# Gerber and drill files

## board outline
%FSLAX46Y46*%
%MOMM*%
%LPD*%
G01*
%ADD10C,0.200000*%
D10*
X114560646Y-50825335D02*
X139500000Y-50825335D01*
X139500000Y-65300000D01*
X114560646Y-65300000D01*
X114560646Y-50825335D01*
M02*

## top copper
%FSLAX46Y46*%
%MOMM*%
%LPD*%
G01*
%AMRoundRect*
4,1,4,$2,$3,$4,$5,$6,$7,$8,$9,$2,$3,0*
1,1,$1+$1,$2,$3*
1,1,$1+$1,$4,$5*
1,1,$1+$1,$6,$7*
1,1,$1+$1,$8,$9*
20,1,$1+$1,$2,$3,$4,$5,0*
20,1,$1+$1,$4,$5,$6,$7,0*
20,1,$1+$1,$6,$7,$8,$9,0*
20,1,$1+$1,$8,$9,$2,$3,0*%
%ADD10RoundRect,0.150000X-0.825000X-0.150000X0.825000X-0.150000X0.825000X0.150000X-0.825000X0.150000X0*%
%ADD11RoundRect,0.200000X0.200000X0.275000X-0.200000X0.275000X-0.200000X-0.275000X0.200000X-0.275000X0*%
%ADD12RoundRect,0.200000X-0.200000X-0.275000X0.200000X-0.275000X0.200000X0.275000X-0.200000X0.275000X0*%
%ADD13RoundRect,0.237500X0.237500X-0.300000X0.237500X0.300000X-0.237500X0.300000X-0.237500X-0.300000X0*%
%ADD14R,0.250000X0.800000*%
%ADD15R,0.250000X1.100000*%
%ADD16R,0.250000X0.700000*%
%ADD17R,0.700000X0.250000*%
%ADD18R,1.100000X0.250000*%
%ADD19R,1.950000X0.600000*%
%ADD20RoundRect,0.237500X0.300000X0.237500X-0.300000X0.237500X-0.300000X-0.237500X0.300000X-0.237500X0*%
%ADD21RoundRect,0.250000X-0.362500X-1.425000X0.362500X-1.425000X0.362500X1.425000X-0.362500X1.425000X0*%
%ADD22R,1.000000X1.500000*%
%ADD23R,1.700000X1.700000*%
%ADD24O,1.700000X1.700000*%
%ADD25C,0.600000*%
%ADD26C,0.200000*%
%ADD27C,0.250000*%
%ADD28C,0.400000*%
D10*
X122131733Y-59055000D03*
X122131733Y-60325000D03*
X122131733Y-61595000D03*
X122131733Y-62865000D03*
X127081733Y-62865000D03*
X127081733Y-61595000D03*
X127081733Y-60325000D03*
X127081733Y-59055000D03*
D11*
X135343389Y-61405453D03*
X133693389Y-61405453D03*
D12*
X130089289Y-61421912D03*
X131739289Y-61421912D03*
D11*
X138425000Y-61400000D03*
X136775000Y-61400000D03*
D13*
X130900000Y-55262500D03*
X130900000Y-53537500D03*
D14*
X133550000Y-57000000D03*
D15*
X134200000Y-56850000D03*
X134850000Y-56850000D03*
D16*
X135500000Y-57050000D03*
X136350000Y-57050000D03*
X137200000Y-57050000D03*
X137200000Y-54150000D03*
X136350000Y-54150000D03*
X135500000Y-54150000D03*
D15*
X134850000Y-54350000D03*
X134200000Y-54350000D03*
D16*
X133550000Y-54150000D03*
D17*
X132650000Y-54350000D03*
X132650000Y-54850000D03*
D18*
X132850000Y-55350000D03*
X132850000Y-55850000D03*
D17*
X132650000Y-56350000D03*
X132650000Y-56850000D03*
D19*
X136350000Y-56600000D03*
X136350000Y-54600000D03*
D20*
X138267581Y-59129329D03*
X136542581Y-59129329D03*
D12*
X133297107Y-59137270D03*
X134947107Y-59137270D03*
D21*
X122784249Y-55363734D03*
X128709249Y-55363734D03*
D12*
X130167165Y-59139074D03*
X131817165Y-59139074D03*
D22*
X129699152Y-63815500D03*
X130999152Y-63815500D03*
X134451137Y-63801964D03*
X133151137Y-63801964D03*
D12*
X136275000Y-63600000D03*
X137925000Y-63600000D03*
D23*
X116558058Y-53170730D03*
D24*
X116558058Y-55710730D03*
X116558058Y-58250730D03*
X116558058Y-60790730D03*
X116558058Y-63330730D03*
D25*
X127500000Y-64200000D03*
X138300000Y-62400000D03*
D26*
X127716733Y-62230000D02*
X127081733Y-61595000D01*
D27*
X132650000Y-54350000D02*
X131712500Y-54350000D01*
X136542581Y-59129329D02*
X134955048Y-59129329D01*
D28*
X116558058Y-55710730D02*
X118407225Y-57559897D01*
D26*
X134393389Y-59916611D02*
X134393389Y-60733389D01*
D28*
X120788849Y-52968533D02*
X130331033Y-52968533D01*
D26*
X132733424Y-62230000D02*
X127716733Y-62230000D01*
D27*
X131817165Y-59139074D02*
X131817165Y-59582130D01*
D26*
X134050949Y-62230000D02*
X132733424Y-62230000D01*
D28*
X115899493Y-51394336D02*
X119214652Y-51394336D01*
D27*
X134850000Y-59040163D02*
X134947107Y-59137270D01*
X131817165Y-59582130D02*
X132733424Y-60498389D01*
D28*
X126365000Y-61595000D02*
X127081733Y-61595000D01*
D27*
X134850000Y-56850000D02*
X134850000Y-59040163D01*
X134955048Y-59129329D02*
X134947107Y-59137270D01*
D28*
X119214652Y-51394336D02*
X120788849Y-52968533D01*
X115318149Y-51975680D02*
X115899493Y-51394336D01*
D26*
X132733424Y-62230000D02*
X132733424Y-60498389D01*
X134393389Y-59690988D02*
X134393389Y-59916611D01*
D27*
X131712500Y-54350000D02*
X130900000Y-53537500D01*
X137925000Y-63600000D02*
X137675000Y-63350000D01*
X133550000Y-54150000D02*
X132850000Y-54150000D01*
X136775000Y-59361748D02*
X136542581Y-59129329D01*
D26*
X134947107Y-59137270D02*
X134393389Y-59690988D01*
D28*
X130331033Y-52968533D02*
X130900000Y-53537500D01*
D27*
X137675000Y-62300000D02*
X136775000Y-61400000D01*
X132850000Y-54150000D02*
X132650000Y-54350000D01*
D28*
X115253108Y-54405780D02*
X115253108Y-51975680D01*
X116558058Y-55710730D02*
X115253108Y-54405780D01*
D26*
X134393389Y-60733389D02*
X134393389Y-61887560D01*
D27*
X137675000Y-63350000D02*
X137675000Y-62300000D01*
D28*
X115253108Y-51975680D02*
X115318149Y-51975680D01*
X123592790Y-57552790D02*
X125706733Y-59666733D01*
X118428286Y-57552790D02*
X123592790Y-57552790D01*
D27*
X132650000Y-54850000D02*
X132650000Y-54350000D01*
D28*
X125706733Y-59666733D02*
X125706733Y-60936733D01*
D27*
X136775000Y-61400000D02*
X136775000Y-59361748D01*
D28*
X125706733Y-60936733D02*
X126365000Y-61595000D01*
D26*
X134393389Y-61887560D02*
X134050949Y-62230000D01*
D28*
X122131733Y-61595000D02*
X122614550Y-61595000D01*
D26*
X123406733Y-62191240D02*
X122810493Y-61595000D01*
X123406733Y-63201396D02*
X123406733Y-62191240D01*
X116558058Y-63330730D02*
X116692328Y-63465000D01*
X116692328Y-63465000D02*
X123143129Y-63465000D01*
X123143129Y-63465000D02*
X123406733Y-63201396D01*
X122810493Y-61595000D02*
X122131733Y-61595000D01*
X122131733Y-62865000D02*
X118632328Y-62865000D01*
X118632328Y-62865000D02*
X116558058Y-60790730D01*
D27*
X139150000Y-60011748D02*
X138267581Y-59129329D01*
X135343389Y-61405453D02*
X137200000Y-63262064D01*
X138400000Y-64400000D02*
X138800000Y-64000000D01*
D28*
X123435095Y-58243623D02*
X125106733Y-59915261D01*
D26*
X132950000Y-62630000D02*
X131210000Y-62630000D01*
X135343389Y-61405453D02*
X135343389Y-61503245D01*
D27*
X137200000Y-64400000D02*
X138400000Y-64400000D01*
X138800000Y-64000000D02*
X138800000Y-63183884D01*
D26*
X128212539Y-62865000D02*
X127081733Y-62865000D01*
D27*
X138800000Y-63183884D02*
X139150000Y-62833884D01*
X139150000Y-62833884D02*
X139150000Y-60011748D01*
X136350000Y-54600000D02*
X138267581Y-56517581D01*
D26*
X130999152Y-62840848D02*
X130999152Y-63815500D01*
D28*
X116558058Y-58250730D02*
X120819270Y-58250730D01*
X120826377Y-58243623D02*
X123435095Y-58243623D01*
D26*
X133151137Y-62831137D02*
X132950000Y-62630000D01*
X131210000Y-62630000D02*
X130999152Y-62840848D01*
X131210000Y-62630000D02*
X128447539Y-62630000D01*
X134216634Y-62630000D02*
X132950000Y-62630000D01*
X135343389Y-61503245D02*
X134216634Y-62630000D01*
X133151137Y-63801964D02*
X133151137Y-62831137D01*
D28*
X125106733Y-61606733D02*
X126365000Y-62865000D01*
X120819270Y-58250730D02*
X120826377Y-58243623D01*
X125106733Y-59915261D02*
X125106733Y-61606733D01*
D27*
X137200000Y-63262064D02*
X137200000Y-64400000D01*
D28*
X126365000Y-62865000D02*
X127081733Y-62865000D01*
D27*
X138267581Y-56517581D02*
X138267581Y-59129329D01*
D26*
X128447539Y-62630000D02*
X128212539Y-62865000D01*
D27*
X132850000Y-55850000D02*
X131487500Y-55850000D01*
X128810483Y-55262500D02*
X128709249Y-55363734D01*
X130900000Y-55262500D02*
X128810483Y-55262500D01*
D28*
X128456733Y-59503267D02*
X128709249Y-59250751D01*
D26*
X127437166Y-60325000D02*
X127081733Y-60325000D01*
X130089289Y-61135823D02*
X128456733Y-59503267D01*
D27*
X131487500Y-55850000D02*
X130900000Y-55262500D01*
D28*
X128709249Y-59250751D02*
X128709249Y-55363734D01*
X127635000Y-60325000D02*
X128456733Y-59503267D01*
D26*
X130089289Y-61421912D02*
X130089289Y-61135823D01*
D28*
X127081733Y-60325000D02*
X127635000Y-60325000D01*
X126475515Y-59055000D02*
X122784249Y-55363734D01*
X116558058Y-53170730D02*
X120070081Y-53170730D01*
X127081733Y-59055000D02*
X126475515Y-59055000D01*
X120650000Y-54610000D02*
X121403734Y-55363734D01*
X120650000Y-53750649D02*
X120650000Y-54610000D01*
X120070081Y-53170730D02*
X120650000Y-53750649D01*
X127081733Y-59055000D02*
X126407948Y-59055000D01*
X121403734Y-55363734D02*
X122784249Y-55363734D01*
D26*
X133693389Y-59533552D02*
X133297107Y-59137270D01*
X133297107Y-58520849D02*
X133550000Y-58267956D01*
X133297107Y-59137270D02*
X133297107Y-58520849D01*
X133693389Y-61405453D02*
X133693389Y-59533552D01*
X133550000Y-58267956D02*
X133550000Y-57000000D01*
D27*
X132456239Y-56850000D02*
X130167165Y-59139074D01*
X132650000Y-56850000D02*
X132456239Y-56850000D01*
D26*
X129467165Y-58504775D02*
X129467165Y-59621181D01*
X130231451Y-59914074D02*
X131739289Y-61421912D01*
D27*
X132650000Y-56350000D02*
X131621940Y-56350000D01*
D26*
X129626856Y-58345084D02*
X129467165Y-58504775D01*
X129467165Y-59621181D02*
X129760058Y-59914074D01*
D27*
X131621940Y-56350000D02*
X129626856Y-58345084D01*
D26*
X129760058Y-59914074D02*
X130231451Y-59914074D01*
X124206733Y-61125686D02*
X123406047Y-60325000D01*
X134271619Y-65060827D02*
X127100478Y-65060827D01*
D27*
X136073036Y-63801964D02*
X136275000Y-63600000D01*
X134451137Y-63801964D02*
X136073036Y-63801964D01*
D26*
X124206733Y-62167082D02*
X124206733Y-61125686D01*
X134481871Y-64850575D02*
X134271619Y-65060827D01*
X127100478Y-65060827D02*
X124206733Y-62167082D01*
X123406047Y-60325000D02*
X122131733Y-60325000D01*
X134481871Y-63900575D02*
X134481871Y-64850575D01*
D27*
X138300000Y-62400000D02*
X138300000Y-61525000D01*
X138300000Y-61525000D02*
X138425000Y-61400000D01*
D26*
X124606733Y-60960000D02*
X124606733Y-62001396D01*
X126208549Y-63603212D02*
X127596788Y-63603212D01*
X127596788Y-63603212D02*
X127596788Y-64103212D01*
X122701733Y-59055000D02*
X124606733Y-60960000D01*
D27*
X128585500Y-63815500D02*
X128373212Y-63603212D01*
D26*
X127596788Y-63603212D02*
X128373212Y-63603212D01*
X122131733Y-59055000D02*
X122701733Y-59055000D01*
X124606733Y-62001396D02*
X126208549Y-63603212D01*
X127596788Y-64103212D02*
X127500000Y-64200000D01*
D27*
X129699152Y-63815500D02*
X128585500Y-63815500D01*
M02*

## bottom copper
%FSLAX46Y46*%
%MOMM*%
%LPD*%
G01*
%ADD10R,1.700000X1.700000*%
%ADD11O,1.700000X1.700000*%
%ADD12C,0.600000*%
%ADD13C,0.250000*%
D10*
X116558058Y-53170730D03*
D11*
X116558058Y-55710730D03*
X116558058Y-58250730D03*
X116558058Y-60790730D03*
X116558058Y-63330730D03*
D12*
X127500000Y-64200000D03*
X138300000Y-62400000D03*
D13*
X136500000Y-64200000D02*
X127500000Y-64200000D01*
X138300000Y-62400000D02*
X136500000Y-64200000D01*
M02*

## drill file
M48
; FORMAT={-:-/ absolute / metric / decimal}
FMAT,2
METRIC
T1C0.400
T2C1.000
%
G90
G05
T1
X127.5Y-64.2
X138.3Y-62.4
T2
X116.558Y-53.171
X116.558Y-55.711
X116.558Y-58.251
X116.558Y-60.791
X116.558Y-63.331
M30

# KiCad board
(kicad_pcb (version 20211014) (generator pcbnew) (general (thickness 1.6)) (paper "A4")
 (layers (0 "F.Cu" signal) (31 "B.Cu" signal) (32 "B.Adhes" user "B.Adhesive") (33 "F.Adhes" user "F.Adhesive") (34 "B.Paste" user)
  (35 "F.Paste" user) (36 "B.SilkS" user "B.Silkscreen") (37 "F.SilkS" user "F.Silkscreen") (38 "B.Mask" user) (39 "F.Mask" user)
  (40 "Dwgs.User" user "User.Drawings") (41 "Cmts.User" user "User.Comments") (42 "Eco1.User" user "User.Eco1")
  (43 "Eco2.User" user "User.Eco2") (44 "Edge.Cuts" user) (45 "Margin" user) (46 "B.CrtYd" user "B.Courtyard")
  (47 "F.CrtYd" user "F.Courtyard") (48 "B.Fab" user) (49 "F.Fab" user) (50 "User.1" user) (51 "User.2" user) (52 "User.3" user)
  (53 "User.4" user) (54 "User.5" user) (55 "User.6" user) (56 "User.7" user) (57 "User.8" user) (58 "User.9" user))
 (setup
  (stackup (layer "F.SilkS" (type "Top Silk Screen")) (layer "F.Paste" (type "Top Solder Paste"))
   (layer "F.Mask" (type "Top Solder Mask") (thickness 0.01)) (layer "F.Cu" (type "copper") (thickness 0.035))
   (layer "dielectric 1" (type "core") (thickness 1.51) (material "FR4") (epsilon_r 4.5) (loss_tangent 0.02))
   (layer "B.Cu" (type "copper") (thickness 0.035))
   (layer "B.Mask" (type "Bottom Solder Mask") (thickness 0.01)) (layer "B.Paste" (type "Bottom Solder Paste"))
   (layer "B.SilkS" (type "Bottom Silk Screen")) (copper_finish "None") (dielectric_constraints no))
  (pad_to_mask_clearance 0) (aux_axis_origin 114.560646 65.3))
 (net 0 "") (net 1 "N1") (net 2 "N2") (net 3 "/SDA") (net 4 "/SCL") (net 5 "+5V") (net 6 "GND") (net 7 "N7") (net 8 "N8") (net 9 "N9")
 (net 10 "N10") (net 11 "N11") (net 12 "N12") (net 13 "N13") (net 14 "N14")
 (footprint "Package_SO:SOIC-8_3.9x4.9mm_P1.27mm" (layer "F.Cu") (at 124.606733 60.96)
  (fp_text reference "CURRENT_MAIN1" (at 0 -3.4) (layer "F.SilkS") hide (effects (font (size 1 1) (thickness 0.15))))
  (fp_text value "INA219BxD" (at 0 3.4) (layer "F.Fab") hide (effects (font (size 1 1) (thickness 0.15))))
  (pad "1" smd roundrect (at -2.475 -1.905) (size 1.95 0.6) (layers "F.Cu" "F.Paste" "F.Mask") (roundrect_rratio 0.25) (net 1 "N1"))
  (pad "2" smd roundrect (at -2.475 -0.635) (size 1.95 0.6) (layers "F.Cu" "F.Paste" "F.Mask") (roundrect_rratio 0.25) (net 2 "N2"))
  (pad "3" smd roundrect (at -2.475 0.635) (size 1.95 0.6) (layers "F.Cu" "F.Paste" "F.Mask") (roundrect_rratio 0.25) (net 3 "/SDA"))
  (pad "4" smd roundrect (at -2.475 1.905) (size 1.95 0.6) (layers "F.Cu" "F.Paste" "F.Mask") (roundrect_rratio 0.25) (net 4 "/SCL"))
  (pad "5" smd roundrect (at 2.475 1.905) (size 1.95 0.6) (layers "F.Cu" "F.Paste" "F.Mask") (roundrect_rratio 0.25) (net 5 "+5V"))
  (pad "6" smd roundrect (at 2.475 0.635) (size 1.95 0.6) (layers "F.Cu" "F.Paste" "F.Mask") (roundrect_rratio 0.25) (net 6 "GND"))
  (pad "7" smd roundrect (at 2.475 -0.635) (size 1.95 0.6) (layers "F.Cu" "F.Paste" "F.Mask") (roundrect_rratio 0.25) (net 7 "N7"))
  (pad "8" smd roundrect (at 2.475 -1.905) (size 1.95 0.6) (layers "F.Cu" "F.Paste" "F.Mask") (roundrect_rratio 0.25) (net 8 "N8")))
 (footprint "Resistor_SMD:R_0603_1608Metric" (layer "F.Cu") (at 134.518389 61.405453 180)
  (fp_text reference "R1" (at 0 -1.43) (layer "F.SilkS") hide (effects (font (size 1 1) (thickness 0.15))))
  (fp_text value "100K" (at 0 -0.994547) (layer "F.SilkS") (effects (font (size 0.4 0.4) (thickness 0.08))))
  (pad "1" smd roundrect (at -0.825 0 180) (size 0.8 0.95) (layers "F.Cu" "F.Paste" "F.Mask") (roundrect_rratio 0.25) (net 5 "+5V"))
  (pad "2" smd roundrect (at 0.825 0 180) (size 0.8 0.95) (layers "F.Cu" "F.Paste" "F.Mask") (roundrect_rratio 0.25) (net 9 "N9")))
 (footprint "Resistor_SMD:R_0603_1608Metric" (layer "F.Cu") (at 130.914289 61.421912)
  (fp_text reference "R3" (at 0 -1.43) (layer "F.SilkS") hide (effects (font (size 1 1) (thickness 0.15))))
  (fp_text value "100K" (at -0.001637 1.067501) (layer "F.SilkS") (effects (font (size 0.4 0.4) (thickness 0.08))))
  (pad "1" smd roundrect (at -0.825 0) (size 0.8 0.95) (layers "F.Cu" "F.Paste" "F.Mask") (roundrect_rratio 0.25) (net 7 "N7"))
  (pad "2" smd roundrect (at 0.825 0) (size 0.8 0.95) (layers "F.Cu" "F.Paste" "F.Mask") (roundrect_rratio 0.25) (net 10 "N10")))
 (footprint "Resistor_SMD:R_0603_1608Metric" (layer "F.Cu") (at 137.6 61.4 180)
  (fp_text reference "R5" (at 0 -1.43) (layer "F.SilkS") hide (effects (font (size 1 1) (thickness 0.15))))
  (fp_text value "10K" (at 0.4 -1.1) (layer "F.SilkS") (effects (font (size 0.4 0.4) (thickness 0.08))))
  (pad "1" smd roundrect (at -0.825 0 180) (size 0.8 0.95) (layers "F.Cu" "F.Paste" "F.Mask") (roundrect_rratio 0.25) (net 1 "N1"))
  (pad "2" smd roundrect (at 0.825 0 180) (size 0.8 0.95) (layers "F.Cu" "F.Paste" "F.Mask") (roundrect_rratio 0.25) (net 6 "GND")))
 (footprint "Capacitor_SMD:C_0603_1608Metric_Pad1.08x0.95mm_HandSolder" (layer "F.Cu") (at 130.9 54.4 90)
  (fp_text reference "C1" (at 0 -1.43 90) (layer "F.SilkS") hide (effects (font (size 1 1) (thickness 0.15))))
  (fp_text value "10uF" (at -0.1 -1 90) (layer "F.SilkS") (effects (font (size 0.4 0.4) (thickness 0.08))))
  (pad "1" smd roundrect (at -0.8625 0 90) (size 1.075 0.95) (layers "F.Cu" "F.Paste" "F.Mask") (roundrect_rratio 0.25) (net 7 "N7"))
  (pad "2" smd roundrect (at 0.8625 0 90) (size 1.075 0.95) (layers "F.Cu" "F.Paste" "F.Mask") (roundrect_rratio 0.25) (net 6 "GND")))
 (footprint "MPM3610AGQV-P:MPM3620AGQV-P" (layer "F.Cu") (at 135.1 55.6 90)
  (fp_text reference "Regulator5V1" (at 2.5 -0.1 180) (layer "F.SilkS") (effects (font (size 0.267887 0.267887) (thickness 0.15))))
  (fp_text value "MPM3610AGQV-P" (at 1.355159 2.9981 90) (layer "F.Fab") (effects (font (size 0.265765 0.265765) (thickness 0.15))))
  (pad "1" smd rect (at -1.4 -1.55 180) (size 0.25 0.8) (layers "F.Cu" "F.Paste" "F.Mask") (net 9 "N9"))
  (pad "2" smd rect (at -1.25 -0.9 180) (size 0.25 1.1) (layers "F.Cu" "F.Paste" "F.Mask") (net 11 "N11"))
  (pad "3" smd rect (at -1.25 -0.25 180) (size 0.25 1.1) (layers "F.Cu" "F.Paste" "F.Mask") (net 6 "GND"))
  (pad "4" smd rect (at -1.45 0.4) (size 0.25 0.7) (layers "F.Cu" "F.Paste" "F.Mask") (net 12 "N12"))
  (pad "5" smd rect (at -1.45 1.25) (size 0.25 0.7) (layers "F.Cu" "F.Paste" "F.Mask") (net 12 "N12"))
  (pad "6" smd rect (at -1.45 2.1) (size 0.25 0.7) (layers "F.Cu" "F.Paste" "F.Mask") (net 12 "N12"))
  (pad "7" smd rect (at 1.45 2.1) (size 0.25 0.7) (layers "F.Cu" "F.Paste" "F.Mask") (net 5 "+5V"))
  (pad "8" smd rect (at 1.45 1.25) (size 0.25 0.7) (layers "F.Cu" "F.Paste" "F.Mask") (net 5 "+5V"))
  (pad "9" smd rect (at 1.45 0.4) (size 0.25 0.7) (layers "F.Cu" "F.Paste" "F.Mask") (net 5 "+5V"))
  (pad "10" smd rect (at 1.25 -0.25 180) (size 0.25 1.1) (layers "F.Cu" "F.Paste" "F.Mask"))
  (pad "11" smd rect (at 1.25 -0.9 180) (size 0.25 1.1) (layers "F.Cu" "F.Paste" "F.Mask") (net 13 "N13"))
  (pad "12" smd rect (at 1.45 -1.55 180) (size 0.25 0.7) (layers "F.Cu" "F.Paste" "F.Mask") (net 6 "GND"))
  (pad "13" smd rect (at 1.25 -2.45 90) (size 0.25 0.7) (layers "F.Cu" "F.Paste" "F.Mask") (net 6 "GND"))
  (pad "14" smd rect (at 0.75 -2.45 90) (size 0.25 0.7) (layers "F.Cu" "F.Paste" "F.Mask") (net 6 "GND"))
  (pad "15" smd rect (at 0.25 -2.25 90) (size 0.25 1.1) (layers "F.Cu" "F.Paste" "F.Mask"))
  (pad "16" smd rect (at -0.25 -2.25 90) (size 0.25 1.1) (layers "F.Cu" "F.Paste" "F.Mask") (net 7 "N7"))
  (pad "17" smd rect (at -0.75 -2.45 90) (size 0.25 0.7) (layers "F.Cu" "F.Paste" "F.Mask") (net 10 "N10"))
  (pad "18" smd rect (at -1.25 -2.45 90) (size 0.25 0.7) (layers "F.Cu" "F.Paste" "F.Mask") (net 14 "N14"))
  (pad "19" smd rect (at -1 1.25 180) (size 1.95 0.6) (layers "F.Cu" "F.Paste" "F.Mask") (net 12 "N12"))
  (pad "20" smd rect (at 1 1.25 180) (size 1.95 0.6) (layers "F.Cu" "F.Paste" "F.Mask") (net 5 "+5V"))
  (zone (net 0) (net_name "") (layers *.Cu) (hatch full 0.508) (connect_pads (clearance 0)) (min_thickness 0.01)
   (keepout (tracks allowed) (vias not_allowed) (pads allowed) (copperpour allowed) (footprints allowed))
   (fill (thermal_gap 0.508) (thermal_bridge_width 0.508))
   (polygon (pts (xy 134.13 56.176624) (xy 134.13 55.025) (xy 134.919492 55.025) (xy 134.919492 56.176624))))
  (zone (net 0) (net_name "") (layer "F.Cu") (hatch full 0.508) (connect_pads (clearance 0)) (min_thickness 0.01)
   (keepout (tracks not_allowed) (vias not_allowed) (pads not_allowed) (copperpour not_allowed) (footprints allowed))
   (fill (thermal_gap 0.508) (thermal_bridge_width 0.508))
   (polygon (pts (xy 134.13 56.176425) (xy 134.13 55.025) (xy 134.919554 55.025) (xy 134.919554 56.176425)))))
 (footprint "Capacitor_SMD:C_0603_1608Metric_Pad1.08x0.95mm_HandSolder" (layer "F.Cu") (at 137.405081 59.129329 180)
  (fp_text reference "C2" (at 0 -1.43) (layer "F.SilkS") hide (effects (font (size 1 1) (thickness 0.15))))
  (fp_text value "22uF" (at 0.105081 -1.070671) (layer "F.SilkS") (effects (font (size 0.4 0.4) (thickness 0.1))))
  (pad "1" smd roundrect (at -0.8625 0 180) (size 1.075 0.95) (layers "F.Cu" "F.Paste" "F.Mask") (roundrect_rratio 0.25) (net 5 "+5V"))
  (pad "2" smd roundrect (at 0.8625 0 180) (size 1.075 0.95) (layers "F.Cu" "F.Paste" "F.Mask") (roundrect_rratio 0.25) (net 6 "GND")))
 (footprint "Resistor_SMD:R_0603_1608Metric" (layer "F.Cu") (at 134.122107 59.13727)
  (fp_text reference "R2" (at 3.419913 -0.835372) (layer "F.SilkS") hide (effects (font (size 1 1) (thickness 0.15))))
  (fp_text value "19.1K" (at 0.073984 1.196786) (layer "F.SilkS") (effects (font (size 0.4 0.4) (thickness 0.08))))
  (pad "1" smd roundrect (at -0.825 0) (size 0.8 0.95) (layers "F.Cu" "F.Paste" "F.Mask") (roundrect_rratio 0.25) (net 9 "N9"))
  (pad "2" smd roundrect (at 0.825 0) (size 0.8 0.95) (layers "F.Cu" "F.Paste" "F.Mask") (roundrect_rratio 0.25) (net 6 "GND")))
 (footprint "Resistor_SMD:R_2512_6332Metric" (layer "F.Cu") (at 125.746749 55.363734)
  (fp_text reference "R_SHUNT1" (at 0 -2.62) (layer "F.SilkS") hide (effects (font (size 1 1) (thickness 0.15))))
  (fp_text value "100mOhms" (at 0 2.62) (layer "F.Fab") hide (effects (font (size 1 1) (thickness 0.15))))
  (pad "1" smd roundrect (at -2.9625 0) (size 1.225 3.35) (layers "F.Cu" "F.Paste" "F.Mask") (roundrect_rratio 0.2040816327) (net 8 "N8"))
  (pad "2" smd roundrect (at 2.9625 0) (size 1.225 3.35) (layers "F.Cu" "F.Paste" "F.Mask") (roundrect_rratio 0.2040816327) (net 7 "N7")))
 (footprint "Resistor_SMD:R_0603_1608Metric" (layer "F.Cu") (at 130.992165 59.139074)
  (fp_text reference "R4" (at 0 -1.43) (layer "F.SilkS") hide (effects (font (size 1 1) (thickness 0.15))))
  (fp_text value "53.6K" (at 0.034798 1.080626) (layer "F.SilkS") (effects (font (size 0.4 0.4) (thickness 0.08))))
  (pad "1" smd roundrect (at -0.825 0) (size 0.8 0.95) (layers "F.Cu" "F.Paste" "F.Mask") (roundrect_rratio 0.25) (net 14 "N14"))
  (pad "2" smd roundrect (at 0.825 0) (size 0.8 0.95) (layers "F.Cu" "F.Paste" "F.Mask") (roundrect_rratio 0.25) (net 6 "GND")))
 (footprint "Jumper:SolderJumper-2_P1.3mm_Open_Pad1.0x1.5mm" (layer "F.Cu") (at 130.349152 63.8155)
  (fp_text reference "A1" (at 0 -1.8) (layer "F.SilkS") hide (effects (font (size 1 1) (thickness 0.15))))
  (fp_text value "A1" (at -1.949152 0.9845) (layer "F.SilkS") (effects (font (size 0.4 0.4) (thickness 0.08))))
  (pad "1" smd rect (at -0.65 0) (size 1 1.5) (layers "F.Cu" "F.Mask") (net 1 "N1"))
  (pad "2" smd rect (at 0.65 0) (size 1 1.5) (layers "F.Cu" "F.Mask") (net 5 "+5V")))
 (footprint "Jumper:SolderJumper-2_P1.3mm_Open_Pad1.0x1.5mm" (layer "F.Cu") (at 133.801137 63.801964 180)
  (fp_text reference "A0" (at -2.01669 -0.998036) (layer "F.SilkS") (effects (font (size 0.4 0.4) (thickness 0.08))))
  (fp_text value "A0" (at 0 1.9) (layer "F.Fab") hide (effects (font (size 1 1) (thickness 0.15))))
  (pad "1" smd rect (at -0.65 0 180) (size 1 1.5) (layers "F.Cu" "F.Mask") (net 2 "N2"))
  (pad "2" smd rect (at 0.65 0 180) (size 1 1.5) (layers "F.Cu" "F.Mask") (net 5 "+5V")))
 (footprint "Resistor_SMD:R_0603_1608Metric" (layer "F.Cu") (at 137.1 63.6)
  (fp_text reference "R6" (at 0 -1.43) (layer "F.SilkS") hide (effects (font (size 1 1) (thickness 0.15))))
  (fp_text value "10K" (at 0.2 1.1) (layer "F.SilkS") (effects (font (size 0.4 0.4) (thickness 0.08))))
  (pad "1" smd roundrect (at -0.825 0) (size 0.8 0.95) (layers "F.Cu" "F.Paste" "F.Mask") (roundrect_rratio 0.25) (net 2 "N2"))
  (pad "2" smd roundrect (at 0.825 0) (size 0.8 0.95) (layers "F.Cu" "F.Paste" "F.Mask") (roundrect_rratio 0.25) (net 6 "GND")))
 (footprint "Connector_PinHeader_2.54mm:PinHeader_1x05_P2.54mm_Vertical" (layer "B.Cu") (at 116.558058 53.17073 180)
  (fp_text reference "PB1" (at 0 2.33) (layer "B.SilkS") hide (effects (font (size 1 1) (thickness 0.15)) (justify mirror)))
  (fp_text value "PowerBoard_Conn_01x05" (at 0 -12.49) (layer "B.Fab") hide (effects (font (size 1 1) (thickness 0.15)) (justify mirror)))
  (pad "1" thru_hole rect (at 0 0 180) (size 1.7 1.7) (drill 1) (layers *.Cu *.Mask) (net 8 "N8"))
  (pad "2" thru_hole oval (at 0 -2.54 180) (size 1.7 1.7) (drill 1) (layers *.Cu *.Mask) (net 6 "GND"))
  (pad "3" thru_hole oval (at 0 -5.08 180) (size 1.7 1.7) (drill 1) (layers *.Cu *.Mask) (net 5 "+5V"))
  (pad "4" thru_hole oval (at 0 -7.62 180) (size 1.7 1.7) (drill 1) (layers *.Cu *.Mask) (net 4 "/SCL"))
  (pad "5" thru_hole oval (at 0 -10.16 180) (size 1.7 1.7) (drill 1) (layers *.Cu *.Mask) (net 3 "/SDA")))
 (gr_rect (start 114.560646 65.3) (end 139.5 50.825335) (layer "Edge.Cuts") (width 0.2) (fill none))
 (segment (start 127.716733 62.23) (end 127.081733 61.595) (width 0.2) (layer "F.Cu") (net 6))
 (segment (start 132.65 54.35) (end 131.7125 54.35) (width 0.25) (layer "F.Cu") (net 6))
 (segment (start 136.542581 59.129329) (end 134.955048 59.129329) (width 0.25) (layer "F.Cu") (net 6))
 (segment (start 116.558058 55.71073) (end 118.407225 57.559897) (width 0.4) (layer "F.Cu") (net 6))
 (segment (start 134.393389 59.916611) (end 134.393389 60.733389) (width 0.2) (layer "F.Cu") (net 6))
 (segment (start 120.788849 52.968533) (end 130.331033 52.968533) (width 0.4) (layer "F.Cu") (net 6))
 (segment (start 132.733424 62.23) (end 127.716733 62.23) (width 0.2) (layer "F.Cu") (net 6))
 (segment (start 131.817165 59.139074) (end 131.817165 59.58213) (width 0.25) (layer "F.Cu") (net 6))
 (segment (start 134.050949 62.23) (end 132.733424 62.23) (width 0.2) (layer "F.Cu") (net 6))
 (segment (start 115.899493 51.394336) (end 119.214652 51.394336) (width 0.4) (layer "F.Cu") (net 6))
 (segment (start 134.85 59.040163) (end 134.947107 59.13727) (width 0.25) (layer "F.Cu") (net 6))
 (segment (start 131.817165 59.58213) (end 132.733424 60.498389) (width 0.25) (layer "F.Cu") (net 6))
 (segment (start 126.365 61.595) (end 127.081733 61.595) (width 0.4) (layer "F.Cu") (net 6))
 (segment (start 134.85 56.85) (end 134.85 59.040163) (width 0.25) (layer "F.Cu") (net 6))
 (segment (start 134.955048 59.129329) (end 134.947107 59.13727) (width 0.25) (layer "F.Cu") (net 6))
 (segment (start 119.214652 51.394336) (end 120.788849 52.968533) (width 0.4) (layer "F.Cu") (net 6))
 (segment (start 115.318149 51.97568) (end 115.899493 51.394336) (width 0.4) (layer "F.Cu") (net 6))
 (segment (start 132.733424 62.23) (end 132.733424 60.498389) (width 0.2) (layer "F.Cu") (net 6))
 (segment (start 134.393389 59.690988) (end 134.393389 59.916611) (width 0.2) (layer "F.Cu") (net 6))
 (segment (start 131.7125 54.35) (end 130.9 53.5375) (width 0.25) (layer "F.Cu") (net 6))
 (segment (start 137.925 63.6) (end 137.675 63.35) (width 0.25) (layer "F.Cu") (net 6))
 (segment (start 133.55 54.15) (end 132.85 54.15) (width 0.25) (layer "F.Cu") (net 6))
 (segment (start 136.775 59.361748) (end 136.542581 59.129329) (width 0.25) (layer "F.Cu") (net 6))
 (segment (start 134.947107 59.13727) (end 134.393389 59.690988) (width 0.2) (layer "F.Cu") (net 6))
 (segment (start 130.331033 52.968533) (end 130.9 53.5375) (width 0.4) (layer "F.Cu") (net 6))
 (segment (start 137.675 62.3) (end 136.775 61.4) (width 0.25) (layer "F.Cu") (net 6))
 (segment (start 132.85 54.15) (end 132.65 54.35) (width 0.25) (layer "F.Cu") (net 6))
 (segment (start 115.253108 54.40578) (end 115.253108 51.97568) (width 0.4) (layer "F.Cu") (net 6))
 (segment (start 116.558058 55.71073) (end 115.253108 54.40578) (width 0.4) (layer "F.Cu") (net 6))
 (segment (start 134.393389 60.733389) (end 134.393389 61.88756) (width 0.2) (layer "F.Cu") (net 6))
 (segment (start 137.675 63.35) (end 137.675 62.3) (width 0.25) (layer "F.Cu") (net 6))
 (segment (start 115.253108 51.97568) (end 115.318149 51.97568) (width 0.4) (layer "F.Cu") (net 6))
 (segment (start 123.59279 57.55279) (end 125.706733 59.666733) (width 0.4) (layer "F.Cu") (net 6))
 (segment (start 118.428286 57.55279) (end 123.59279 57.55279) (width 0.4) (layer "F.Cu") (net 6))
 (segment (start 132.65 54.85) (end 132.65 54.35) (width 0.25) (layer "F.Cu") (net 6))
 (segment (start 125.706733 59.666733) (end 125.706733 60.936733) (width 0.4) (layer "F.Cu") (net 6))
 (segment (start 136.775 61.4) (end 136.775 59.361748) (width 0.25) (layer "F.Cu") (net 6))
 (segment (start 125.706733 60.936733) (end 126.365 61.595) (width 0.4) (layer "F.Cu") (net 6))
 (segment (start 134.393389 61.88756) (end 134.050949 62.23) (width 0.2) (layer "F.Cu") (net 6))
 (segment (start 122.131733 61.595) (end 122.61455 61.595) (width 0.4) (layer "F.Cu") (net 3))
 (segment (start 123.406733 62.19124) (end 122.810493 61.595) (width 0.2) (layer "F.Cu") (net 3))
 (segment (start 123.406733 63.201396) (end 123.406733 62.19124) (width 0.2) (layer "F.Cu") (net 3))
 (segment (start 116.558058 63.33073) (end 116.692328 63.465) (width 0.2) (layer "F.Cu") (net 3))
 (segment (start 116.692328 63.465) (end 123.143129 63.465) (width 0.2) (layer "F.Cu") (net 3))
 (segment (start 123.143129 63.465) (end 123.406733 63.201396) (width 0.2) (layer "F.Cu") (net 3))
 (segment (start 122.810493 61.595) (end 122.131733 61.595) (width 0.2) (layer "F.Cu") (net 3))
 (segment (start 122.131733 62.865) (end 118.632328 62.865) (width 0.2) (layer "F.Cu") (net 4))
 (segment (start 118.632328 62.865) (end 116.558058 60.79073) (width 0.2) (layer "F.Cu") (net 4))
 (segment (start 139.15 60.011748) (end 138.267581 59.129329) (width 0.25) (layer "F.Cu") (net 5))
 (segment (start 135.343389 61.405453) (end 137.2 63.262064) (width 0.25) (layer "F.Cu") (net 5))
 (segment (start 138.4 64.4) (end 138.8 64) (width 0.25) (layer "F.Cu") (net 5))
 (segment (start 123.435095 58.243623) (end 125.106733 59.915261) (width 0.4) (layer "F.Cu") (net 5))
 (segment (start 132.95 62.63) (end 131.21 62.63) (width 0.2) (layer "F.Cu") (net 5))
 (segment (start 135.343389 61.405453) (end 135.343389 61.503245) (width 0.2) (layer "F.Cu") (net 5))
 (segment (start 137.2 64.4) (end 138.4 64.4) (width 0.25) (layer "F.Cu") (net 5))
 (segment (start 138.8 64) (end 138.8 63.183884) (width 0.25) (layer "F.Cu") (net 5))
 (segment (start 128.212539 62.865) (end 127.081733 62.865) (width 0.2) (layer "F.Cu") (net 5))
 (segment (start 138.8 63.183884) (end 139.15 62.833884) (width 0.25) (layer "F.Cu") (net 5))
 (segment (start 139.15 62.833884) (end 139.15 60.011748) (width 0.25) (layer "F.Cu") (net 5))
 (segment (start 136.35 54.6) (end 138.267581 56.517581) (width 0.25) (layer "F.Cu") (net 5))
 (segment (start 130.999152 62.840848) (end 130.999152 63.8155) (width 0.2) (layer "F.Cu") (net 5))
 (segment (start 116.558058 58.25073) (end 120.81927 58.25073) (width 0.4) (layer "F.Cu") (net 5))
 (segment (start 120.826377 58.243623) (end 123.435095 58.243623) (width 0.4) (layer "F.Cu") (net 5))
 (segment (start 133.151137 62.831137) (end 132.95 62.63) (width 0.2) (layer "F.Cu") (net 5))
 (segment (start 131.21 62.63) (end 130.999152 62.840848) (width 0.2) (layer "F.Cu") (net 5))
 (segment (start 131.21 62.63) (end 128.447539 62.63) (width 0.2) (layer "F.Cu") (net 5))
 (segment (start 134.216634 62.63) (end 132.95 62.63) (width 0.2) (layer "F.Cu") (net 5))
 (segment (start 135.343389 61.503245) (end 134.216634 62.63) (width 0.2) (layer "F.Cu") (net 5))
 (segment (start 133.151137 63.801964) (end 133.151137 62.831137) (width 0.2) (layer "F.Cu") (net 5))
 (segment (start 125.106733 61.606733) (end 126.365 62.865) (width 0.4) (layer "F.Cu") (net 5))
 (segment (start 120.81927 58.25073) (end 120.826377 58.243623) (width 0.4) (layer "F.Cu") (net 5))
 (segment (start 125.106733 59.915261) (end 125.106733 61.606733) (width 0.4) (layer "F.Cu") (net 5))
 (segment (start 137.2 63.262064) (end 137.2 64.4) (width 0.25) (layer "F.Cu") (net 5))
 (segment (start 126.365 62.865) (end 127.081733 62.865) (width 0.4) (layer "F.Cu") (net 5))
 (segment (start 138.267581 56.517581) (end 138.267581 59.129329) (width 0.25) (layer "F.Cu") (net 5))
 (segment (start 128.447539 62.63) (end 128.212539 62.865) (width 0.2) (layer "F.Cu") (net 5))
 (segment (start 132.85 55.85) (end 131.4875 55.85) (width 0.25) (layer "F.Cu") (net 7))
 (segment (start 128.810483 55.2625) (end 128.709249 55.363734) (width 0.25) (layer "F.Cu") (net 7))
 (segment (start 130.9 55.2625) (end 128.810483 55.2625) (width 0.25) (layer "F.Cu") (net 7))
 (segment (start 128.456733 59.503267) (end 128.709249 59.250751) (width 0.4) (layer "F.Cu") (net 7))
 (segment (start 127.437166 60.325) (end 127.081733 60.325) (width 0.2) (layer "F.Cu") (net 7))
 (segment (start 130.089289 61.135823) (end 128.456733 59.503267) (width 0.2) (layer "F.Cu") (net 7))
 (segment (start 131.4875 55.85) (end 130.9 55.2625) (width 0.25) (layer "F.Cu") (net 7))
 (segment (start 128.709249 59.250751) (end 128.709249 55.363734) (width 0.4) (layer "F.Cu") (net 7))
 (segment (start 127.635 60.325) (end 128.456733 59.503267) (width 0.4) (layer "F.Cu") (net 7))
 (segment (start 130.089289 61.421912) (end 130.089289 61.135823) (width 0.2) (layer "F.Cu") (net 7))
 (segment (start 127.081733 60.325) (end 127.635 60.325) (width 0.4) (layer "F.Cu") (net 7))
 (segment (start 126.475515 59.055) (end 122.784249 55.363734) (width 0.4) (layer "F.Cu") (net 8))
 (segment (start 116.558058 53.17073) (end 120.070081 53.17073) (width 0.4) (layer "F.Cu") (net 8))
 (segment (start 127.081733 59.055) (end 126.475515 59.055) (width 0.4) (layer "F.Cu") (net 8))
 (segment (start 120.65 54.61) (end 121.403734 55.363734) (width 0.4) (layer "F.Cu") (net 8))
 (segment (start 120.65 53.750649) (end 120.65 54.61) (width 0.4) (layer "F.Cu") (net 8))
 (segment (start 120.070081 53.17073) (end 120.65 53.750649) (width 0.4) (layer "F.Cu") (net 8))
 (segment (start 127.081733 59.055) (end 126.407948 59.055) (width 0.4) (layer "F.Cu") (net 8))
 (segment (start 121.403734 55.363734) (end 122.784249 55.363734) (width 0.4) (layer "F.Cu") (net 8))
 (segment (start 133.693389 59.533552) (end 133.297107 59.13727) (width 0.2) (layer "F.Cu") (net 9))
 (segment (start 133.297107 58.520849) (end 133.55 58.267956) (width 0.2) (layer "F.Cu") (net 9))
 (segment (start 133.297107 59.13727) (end 133.297107 58.520849) (width 0.2) (layer "F.Cu") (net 9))
 (segment (start 133.693389 61.405453) (end 133.693389 59.533552) (width 0.2) (layer "F.Cu") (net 9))
 (segment (start 133.55 58.267956) (end 133.55 57) (width 0.2) (layer "F.Cu") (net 9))
 (segment (start 132.456239 56.85) (end 130.167165 59.139074) (width 0.25) (layer "F.Cu") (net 14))
 (segment (start 132.65 56.85) (end 132.456239 56.85) (width 0.25) (layer "F.Cu") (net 14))
 (segment (start 129.467165 58.504775) (end 129.467165 59.621181) (width 0.2) (layer "F.Cu") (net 10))
 (segment (start 130.231451 59.914074) (end 131.739289 61.421912) (width 0.2) (layer "F.Cu") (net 10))
 (segment (start 132.65 56.35) (end 131.62194 56.35) (width 0.25) (layer "F.Cu") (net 10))
 (segment (start 129.626856 58.345084) (end 129.467165 58.504775) (width 0.2) (layer "F.Cu") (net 10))
 (segment (start 129.467165 59.621181) (end 129.760058 59.914074) (width 0.2) (layer "F.Cu") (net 10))
 (segment (start 131.62194 56.35) (end 129.626856 58.345084) (width 0.25) (layer "F.Cu") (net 10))
 (segment (start 129.760058 59.914074) (end 130.231451 59.914074) (width 0.2) (layer "F.Cu") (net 10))
 (segment (start 124.206733 61.125686) (end 123.406047 60.325) (width 0.2) (layer "F.Cu") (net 2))
 (segment (start 134.271619 65.060827) (end 127.100478 65.060827) (width 0.2) (layer "F.Cu") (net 2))
 (segment (start 136.073036 63.801964) (end 136.275 63.6) (width 0.25) (layer "F.Cu") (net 2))
 (segment (start 134.451137 63.801964) (end 136.073036 63.801964) (width 0.25) (layer "F.Cu") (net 2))
 (segment (start 124.206733 62.167082) (end 124.206733 61.125686) (width 0.2) (layer "F.Cu") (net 2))
 (segment (start 134.481871 64.850575) (end 134.271619 65.060827) (width 0.2) (layer "F.Cu") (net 2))
 (segment (start 127.100478 65.060827) (end 124.206733 62.167082) (width 0.2) (layer "F.Cu") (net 2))
 (segment (start 123.406047 60.325) (end 122.131733 60.325) (width 0.2) (layer "F.Cu") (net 2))
 (segment (start 134.481871 63.900575) (end 134.481871 64.850575) (width 0.2) (layer "F.Cu") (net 2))
 (segment (start 138.3 62.4) (end 138.3 61.525) (width 0.25) (layer "F.Cu") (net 1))
 (segment (start 138.3 61.525) (end 138.425 61.4) (width 0.25) (layer "F.Cu") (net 1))
 (segment (start 124.606733 60.96) (end 124.606733 62.001396) (width 0.2) (layer "F.Cu") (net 1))
 (segment (start 126.208549 63.603212) (end 127.596788 63.603212) (width 0.2) (layer "F.Cu") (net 1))
 (segment (start 127.596788 63.603212) (end 127.596788 64.103212) (width 0.2) (layer "F.Cu") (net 1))
 (segment (start 122.701733 59.055) (end 124.606733 60.96) (width 0.2) (layer "F.Cu") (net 1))
 (segment (start 128.5855 63.8155) (end 128.373212 63.603212) (width 0.25) (layer "F.Cu") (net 1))
 (segment (start 127.596788 63.603212) (end 128.373212 63.603212) (width 0.2) (layer "F.Cu") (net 1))
 (segment (start 122.131733 59.055) (end 122.701733 59.055) (width 0.2) (layer "F.Cu") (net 1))
 (segment (start 124.606733 62.001396) (end 126.208549 63.603212) (width 0.2) (layer "F.Cu") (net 1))
 (segment (start 127.596788 64.103212) (end 127.5 64.2) (width 0.2) (layer "F.Cu") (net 1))
 (segment (start 129.699152 63.8155) (end 128.5855 63.8155) (width 0.25) (layer "F.Cu") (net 1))
 (via (at 127.5 64.2) (size 0.6) (drill 0.4) (layers "F.Cu" "B.Cu") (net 1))
 (via (at 138.3 62.4) (size 0.6) (drill 0.4) (layers "F.Cu" "B.Cu") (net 1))
 (segment (start 136.5 64.2) (end 127.5 64.2) (width 0.25) (layer "B.Cu") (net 1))
 (segment (start 138.3 62.4) (end 136.5 64.2) (width 0.25) (layer "B.Cu") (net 1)))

